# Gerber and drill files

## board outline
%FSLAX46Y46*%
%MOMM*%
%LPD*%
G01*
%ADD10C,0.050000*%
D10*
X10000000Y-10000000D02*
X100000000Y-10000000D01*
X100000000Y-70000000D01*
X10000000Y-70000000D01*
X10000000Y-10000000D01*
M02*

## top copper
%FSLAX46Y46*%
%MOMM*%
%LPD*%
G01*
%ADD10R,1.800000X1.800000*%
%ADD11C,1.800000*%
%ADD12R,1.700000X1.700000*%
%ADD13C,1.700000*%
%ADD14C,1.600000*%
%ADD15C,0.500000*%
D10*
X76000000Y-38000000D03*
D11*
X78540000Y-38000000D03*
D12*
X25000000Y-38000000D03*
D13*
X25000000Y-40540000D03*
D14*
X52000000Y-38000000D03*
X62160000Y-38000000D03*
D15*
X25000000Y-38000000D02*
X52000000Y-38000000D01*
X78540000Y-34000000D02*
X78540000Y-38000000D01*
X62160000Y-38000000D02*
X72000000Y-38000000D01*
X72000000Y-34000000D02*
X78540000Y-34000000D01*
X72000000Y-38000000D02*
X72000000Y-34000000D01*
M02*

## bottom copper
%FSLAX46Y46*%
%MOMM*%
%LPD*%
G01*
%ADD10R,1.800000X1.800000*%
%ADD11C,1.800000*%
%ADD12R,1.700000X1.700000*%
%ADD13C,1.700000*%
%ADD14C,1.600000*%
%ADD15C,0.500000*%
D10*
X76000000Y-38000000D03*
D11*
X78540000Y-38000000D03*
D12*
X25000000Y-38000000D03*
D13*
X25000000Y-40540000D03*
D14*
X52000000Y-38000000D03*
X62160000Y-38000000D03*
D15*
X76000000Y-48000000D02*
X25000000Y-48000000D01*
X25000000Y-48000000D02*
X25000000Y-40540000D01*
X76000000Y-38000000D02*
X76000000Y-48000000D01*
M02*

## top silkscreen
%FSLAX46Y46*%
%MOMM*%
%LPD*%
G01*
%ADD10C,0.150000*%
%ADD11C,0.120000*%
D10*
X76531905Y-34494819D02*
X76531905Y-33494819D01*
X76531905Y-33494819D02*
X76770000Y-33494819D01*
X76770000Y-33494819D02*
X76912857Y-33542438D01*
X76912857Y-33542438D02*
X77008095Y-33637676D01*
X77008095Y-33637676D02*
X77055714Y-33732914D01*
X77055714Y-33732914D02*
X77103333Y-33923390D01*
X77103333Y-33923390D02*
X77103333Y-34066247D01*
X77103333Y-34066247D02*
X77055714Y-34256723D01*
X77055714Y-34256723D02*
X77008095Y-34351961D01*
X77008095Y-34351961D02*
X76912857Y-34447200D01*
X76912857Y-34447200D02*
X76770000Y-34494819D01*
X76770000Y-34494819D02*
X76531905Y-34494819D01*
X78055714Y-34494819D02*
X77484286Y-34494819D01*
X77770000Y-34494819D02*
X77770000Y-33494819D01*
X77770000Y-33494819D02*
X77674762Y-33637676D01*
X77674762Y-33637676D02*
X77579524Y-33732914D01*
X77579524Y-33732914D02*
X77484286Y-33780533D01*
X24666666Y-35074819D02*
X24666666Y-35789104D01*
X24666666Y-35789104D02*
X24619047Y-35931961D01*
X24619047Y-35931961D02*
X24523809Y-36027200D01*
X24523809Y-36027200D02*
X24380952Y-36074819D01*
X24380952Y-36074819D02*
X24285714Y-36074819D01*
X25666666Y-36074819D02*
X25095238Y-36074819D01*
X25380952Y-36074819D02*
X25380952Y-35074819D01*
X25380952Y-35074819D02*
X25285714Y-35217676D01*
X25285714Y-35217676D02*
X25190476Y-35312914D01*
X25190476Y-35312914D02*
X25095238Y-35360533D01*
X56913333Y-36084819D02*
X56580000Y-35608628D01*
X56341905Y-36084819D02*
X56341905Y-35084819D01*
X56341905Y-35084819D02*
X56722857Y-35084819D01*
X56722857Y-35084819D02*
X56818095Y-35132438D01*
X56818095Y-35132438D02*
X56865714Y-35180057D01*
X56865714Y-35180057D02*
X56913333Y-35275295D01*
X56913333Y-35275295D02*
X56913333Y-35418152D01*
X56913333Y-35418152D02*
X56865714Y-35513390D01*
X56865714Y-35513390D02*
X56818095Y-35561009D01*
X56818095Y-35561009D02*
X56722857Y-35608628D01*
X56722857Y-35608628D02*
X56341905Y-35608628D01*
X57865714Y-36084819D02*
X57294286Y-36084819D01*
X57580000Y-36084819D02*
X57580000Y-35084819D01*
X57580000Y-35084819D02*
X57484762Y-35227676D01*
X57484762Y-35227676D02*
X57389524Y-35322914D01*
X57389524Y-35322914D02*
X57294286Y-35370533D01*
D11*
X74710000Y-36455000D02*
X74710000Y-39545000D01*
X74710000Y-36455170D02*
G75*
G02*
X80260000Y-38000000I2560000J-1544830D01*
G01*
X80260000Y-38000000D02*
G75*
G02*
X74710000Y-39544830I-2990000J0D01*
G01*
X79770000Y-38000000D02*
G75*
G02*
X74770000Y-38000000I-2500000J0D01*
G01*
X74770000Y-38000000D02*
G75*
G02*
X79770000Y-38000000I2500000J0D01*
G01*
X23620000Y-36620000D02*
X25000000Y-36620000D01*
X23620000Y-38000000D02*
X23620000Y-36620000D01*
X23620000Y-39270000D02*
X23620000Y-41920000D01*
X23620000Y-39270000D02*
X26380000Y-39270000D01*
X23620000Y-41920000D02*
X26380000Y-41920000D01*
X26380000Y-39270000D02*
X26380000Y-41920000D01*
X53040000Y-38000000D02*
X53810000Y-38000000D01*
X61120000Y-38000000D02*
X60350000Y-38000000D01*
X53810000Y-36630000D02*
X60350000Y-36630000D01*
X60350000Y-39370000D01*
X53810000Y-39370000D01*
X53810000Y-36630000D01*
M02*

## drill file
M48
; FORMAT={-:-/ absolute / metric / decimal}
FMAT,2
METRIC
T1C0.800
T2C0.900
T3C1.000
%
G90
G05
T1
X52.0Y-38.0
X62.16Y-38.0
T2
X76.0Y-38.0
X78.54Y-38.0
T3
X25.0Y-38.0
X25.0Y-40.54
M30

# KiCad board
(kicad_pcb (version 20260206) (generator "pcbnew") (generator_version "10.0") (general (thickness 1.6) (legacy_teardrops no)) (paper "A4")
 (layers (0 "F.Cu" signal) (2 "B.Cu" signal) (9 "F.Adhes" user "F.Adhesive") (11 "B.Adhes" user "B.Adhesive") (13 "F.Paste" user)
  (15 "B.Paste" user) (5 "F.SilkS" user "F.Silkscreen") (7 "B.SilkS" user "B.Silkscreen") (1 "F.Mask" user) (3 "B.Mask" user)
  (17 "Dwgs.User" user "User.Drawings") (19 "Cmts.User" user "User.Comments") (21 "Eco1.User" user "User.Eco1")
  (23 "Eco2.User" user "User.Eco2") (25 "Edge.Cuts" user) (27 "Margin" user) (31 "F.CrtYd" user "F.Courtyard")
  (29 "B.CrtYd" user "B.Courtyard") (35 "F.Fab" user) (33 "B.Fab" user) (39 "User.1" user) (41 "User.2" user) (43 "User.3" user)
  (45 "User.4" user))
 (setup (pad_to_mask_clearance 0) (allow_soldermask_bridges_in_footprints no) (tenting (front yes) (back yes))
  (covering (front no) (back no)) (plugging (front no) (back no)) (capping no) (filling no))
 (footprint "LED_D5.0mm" (layer "F.Cu") (at 76 38)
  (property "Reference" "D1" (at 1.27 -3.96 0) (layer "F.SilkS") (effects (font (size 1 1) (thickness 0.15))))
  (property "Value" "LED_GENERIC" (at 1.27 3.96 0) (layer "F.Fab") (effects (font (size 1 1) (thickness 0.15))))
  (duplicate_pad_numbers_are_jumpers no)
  (fp_line (start -1.29 -1.545) (end -1.29 1.545) (stroke (width 0.12) (type solid)) (layer "F.SilkS"))
  (fp_arc (start -1.29 -1.54483) (mid 2.071779 -2.880495) (end 4.26 0) (stroke (width 0.12) (type solid)) (layer "F.SilkS"))
  (fp_arc (start 4.26 0) (mid 2.071779 2.880495) (end -1.29 1.54483) (stroke (width 0.12) (type solid)) (layer "F.SilkS"))
  (fp_circle (center 1.27 0) (end 3.77 0) (stroke (width 0.12) (type solid)) (fill no) (layer "F.SilkS"))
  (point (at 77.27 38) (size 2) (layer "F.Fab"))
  (pad "1" thru_hole rect (at 0 0) (size 1.8 1.8) (drill 0.9) (layers "*.Cu" "*.Mask") (remove_unused_layers no) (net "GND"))
  (pad "2" thru_hole circle (at 2.54 0) (size 1.8 1.8) (drill 0.9) (layers "*.Cu" "*.Mask") (remove_unused_layers no) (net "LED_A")))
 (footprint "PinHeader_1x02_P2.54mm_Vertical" (layer "F.Cu") (at 25 38)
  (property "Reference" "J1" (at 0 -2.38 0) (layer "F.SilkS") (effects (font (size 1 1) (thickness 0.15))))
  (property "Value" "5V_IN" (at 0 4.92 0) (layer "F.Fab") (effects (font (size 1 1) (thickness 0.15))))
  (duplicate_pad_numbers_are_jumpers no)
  (fp_line (start -1.38 -1.38) (end 0 -1.38) (stroke (width 0.12) (type solid)) (layer "F.SilkS"))
  (fp_line (start -1.38 0) (end -1.38 -1.38) (stroke (width 0.12) (type solid)) (layer "F.SilkS"))
  (fp_line (start -1.38 1.27) (end -1.38 3.92) (stroke (width 0.12) (type solid)) (layer "F.SilkS"))
  (fp_line (start -1.38 1.27) (end 1.38 1.27) (stroke (width 0.12) (type solid)) (layer "F.SilkS"))
  (fp_line (start -1.38 3.92) (end 1.38 3.92) (stroke (width 0.12) (type solid)) (layer "F.SilkS"))
  (fp_line (start 1.38 1.27) (end 1.38 3.92) (stroke (width 0.12) (type solid)) (layer "F.SilkS"))
  (pad "1" thru_hole rect (at 0 0) (size 1.7 1.7) (drill 1) (layers "*.Cu" "*.Mask") (remove_unused_layers no) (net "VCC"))
  (pad "2" thru_hole circle (at 0 2.54) (size 1.7 1.7) (drill 1) (layers "*.Cu" "*.Mask") (remove_unused_layers no) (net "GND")))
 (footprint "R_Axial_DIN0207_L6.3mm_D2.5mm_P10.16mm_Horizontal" (layer "F.Cu") (at 52 38)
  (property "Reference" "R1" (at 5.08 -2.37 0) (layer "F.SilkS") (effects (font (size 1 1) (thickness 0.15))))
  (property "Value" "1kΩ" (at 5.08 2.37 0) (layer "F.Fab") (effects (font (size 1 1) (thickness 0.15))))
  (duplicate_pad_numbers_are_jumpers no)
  (fp_line (start 1.04 0) (end 1.81 0) (stroke (width 0.12) (type solid)) (layer "F.SilkS"))
  (fp_line (start 9.12 0) (end 8.35 0) (stroke (width 0.12) (type solid)) (layer "F.SilkS"))
  (fp_rect (start 1.81 -1.37) (end 8.35 1.37) (stroke (width 0.12) (type solid)) (fill no) (layer "F.SilkS"))
  (pad "1" thru_hole circle (at 0 0) (size 1.6 1.6) (drill 0.8) (layers "*.Cu" "*.Mask") (remove_unused_layers no) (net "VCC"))
  (pad "2" thru_hole circle (at 10.16 0) (size 1.6 1.6) (drill 0.8) (layers "*.Cu" "*.Mask") (remove_unused_layers no) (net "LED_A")))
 (gr_rect (start 10 10) (end 100 70) (stroke (width 0.05) (type default)) (fill no) (layer "Edge.Cuts"))
 (segment (start 25 38) (end 52 38) (width 0.5) (layer "F.Cu") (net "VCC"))
 (segment (start 78.54 34) (end 78.54 38) (width 0.5) (layer "F.Cu") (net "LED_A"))
 (segment (start 62.16 38) (end 72 38) (width 0.5) (layer "F.Cu") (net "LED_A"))
 (segment (start 72 34) (end 78.54 34) (width 0.5) (layer "F.Cu") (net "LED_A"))
 (segment (start 72 38) (end 72 34) (width 0.5) (layer "F.Cu") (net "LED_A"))
 (segment (start 76 48) (end 25 48) (width 0.5) (layer "B.Cu") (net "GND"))
 (segment (start 25 48) (end 25 40.54) (width 0.5) (layer "B.Cu") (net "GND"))
 (segment (start 76 38) (end 76 48) (width 0.5) (layer "B.Cu") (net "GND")))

